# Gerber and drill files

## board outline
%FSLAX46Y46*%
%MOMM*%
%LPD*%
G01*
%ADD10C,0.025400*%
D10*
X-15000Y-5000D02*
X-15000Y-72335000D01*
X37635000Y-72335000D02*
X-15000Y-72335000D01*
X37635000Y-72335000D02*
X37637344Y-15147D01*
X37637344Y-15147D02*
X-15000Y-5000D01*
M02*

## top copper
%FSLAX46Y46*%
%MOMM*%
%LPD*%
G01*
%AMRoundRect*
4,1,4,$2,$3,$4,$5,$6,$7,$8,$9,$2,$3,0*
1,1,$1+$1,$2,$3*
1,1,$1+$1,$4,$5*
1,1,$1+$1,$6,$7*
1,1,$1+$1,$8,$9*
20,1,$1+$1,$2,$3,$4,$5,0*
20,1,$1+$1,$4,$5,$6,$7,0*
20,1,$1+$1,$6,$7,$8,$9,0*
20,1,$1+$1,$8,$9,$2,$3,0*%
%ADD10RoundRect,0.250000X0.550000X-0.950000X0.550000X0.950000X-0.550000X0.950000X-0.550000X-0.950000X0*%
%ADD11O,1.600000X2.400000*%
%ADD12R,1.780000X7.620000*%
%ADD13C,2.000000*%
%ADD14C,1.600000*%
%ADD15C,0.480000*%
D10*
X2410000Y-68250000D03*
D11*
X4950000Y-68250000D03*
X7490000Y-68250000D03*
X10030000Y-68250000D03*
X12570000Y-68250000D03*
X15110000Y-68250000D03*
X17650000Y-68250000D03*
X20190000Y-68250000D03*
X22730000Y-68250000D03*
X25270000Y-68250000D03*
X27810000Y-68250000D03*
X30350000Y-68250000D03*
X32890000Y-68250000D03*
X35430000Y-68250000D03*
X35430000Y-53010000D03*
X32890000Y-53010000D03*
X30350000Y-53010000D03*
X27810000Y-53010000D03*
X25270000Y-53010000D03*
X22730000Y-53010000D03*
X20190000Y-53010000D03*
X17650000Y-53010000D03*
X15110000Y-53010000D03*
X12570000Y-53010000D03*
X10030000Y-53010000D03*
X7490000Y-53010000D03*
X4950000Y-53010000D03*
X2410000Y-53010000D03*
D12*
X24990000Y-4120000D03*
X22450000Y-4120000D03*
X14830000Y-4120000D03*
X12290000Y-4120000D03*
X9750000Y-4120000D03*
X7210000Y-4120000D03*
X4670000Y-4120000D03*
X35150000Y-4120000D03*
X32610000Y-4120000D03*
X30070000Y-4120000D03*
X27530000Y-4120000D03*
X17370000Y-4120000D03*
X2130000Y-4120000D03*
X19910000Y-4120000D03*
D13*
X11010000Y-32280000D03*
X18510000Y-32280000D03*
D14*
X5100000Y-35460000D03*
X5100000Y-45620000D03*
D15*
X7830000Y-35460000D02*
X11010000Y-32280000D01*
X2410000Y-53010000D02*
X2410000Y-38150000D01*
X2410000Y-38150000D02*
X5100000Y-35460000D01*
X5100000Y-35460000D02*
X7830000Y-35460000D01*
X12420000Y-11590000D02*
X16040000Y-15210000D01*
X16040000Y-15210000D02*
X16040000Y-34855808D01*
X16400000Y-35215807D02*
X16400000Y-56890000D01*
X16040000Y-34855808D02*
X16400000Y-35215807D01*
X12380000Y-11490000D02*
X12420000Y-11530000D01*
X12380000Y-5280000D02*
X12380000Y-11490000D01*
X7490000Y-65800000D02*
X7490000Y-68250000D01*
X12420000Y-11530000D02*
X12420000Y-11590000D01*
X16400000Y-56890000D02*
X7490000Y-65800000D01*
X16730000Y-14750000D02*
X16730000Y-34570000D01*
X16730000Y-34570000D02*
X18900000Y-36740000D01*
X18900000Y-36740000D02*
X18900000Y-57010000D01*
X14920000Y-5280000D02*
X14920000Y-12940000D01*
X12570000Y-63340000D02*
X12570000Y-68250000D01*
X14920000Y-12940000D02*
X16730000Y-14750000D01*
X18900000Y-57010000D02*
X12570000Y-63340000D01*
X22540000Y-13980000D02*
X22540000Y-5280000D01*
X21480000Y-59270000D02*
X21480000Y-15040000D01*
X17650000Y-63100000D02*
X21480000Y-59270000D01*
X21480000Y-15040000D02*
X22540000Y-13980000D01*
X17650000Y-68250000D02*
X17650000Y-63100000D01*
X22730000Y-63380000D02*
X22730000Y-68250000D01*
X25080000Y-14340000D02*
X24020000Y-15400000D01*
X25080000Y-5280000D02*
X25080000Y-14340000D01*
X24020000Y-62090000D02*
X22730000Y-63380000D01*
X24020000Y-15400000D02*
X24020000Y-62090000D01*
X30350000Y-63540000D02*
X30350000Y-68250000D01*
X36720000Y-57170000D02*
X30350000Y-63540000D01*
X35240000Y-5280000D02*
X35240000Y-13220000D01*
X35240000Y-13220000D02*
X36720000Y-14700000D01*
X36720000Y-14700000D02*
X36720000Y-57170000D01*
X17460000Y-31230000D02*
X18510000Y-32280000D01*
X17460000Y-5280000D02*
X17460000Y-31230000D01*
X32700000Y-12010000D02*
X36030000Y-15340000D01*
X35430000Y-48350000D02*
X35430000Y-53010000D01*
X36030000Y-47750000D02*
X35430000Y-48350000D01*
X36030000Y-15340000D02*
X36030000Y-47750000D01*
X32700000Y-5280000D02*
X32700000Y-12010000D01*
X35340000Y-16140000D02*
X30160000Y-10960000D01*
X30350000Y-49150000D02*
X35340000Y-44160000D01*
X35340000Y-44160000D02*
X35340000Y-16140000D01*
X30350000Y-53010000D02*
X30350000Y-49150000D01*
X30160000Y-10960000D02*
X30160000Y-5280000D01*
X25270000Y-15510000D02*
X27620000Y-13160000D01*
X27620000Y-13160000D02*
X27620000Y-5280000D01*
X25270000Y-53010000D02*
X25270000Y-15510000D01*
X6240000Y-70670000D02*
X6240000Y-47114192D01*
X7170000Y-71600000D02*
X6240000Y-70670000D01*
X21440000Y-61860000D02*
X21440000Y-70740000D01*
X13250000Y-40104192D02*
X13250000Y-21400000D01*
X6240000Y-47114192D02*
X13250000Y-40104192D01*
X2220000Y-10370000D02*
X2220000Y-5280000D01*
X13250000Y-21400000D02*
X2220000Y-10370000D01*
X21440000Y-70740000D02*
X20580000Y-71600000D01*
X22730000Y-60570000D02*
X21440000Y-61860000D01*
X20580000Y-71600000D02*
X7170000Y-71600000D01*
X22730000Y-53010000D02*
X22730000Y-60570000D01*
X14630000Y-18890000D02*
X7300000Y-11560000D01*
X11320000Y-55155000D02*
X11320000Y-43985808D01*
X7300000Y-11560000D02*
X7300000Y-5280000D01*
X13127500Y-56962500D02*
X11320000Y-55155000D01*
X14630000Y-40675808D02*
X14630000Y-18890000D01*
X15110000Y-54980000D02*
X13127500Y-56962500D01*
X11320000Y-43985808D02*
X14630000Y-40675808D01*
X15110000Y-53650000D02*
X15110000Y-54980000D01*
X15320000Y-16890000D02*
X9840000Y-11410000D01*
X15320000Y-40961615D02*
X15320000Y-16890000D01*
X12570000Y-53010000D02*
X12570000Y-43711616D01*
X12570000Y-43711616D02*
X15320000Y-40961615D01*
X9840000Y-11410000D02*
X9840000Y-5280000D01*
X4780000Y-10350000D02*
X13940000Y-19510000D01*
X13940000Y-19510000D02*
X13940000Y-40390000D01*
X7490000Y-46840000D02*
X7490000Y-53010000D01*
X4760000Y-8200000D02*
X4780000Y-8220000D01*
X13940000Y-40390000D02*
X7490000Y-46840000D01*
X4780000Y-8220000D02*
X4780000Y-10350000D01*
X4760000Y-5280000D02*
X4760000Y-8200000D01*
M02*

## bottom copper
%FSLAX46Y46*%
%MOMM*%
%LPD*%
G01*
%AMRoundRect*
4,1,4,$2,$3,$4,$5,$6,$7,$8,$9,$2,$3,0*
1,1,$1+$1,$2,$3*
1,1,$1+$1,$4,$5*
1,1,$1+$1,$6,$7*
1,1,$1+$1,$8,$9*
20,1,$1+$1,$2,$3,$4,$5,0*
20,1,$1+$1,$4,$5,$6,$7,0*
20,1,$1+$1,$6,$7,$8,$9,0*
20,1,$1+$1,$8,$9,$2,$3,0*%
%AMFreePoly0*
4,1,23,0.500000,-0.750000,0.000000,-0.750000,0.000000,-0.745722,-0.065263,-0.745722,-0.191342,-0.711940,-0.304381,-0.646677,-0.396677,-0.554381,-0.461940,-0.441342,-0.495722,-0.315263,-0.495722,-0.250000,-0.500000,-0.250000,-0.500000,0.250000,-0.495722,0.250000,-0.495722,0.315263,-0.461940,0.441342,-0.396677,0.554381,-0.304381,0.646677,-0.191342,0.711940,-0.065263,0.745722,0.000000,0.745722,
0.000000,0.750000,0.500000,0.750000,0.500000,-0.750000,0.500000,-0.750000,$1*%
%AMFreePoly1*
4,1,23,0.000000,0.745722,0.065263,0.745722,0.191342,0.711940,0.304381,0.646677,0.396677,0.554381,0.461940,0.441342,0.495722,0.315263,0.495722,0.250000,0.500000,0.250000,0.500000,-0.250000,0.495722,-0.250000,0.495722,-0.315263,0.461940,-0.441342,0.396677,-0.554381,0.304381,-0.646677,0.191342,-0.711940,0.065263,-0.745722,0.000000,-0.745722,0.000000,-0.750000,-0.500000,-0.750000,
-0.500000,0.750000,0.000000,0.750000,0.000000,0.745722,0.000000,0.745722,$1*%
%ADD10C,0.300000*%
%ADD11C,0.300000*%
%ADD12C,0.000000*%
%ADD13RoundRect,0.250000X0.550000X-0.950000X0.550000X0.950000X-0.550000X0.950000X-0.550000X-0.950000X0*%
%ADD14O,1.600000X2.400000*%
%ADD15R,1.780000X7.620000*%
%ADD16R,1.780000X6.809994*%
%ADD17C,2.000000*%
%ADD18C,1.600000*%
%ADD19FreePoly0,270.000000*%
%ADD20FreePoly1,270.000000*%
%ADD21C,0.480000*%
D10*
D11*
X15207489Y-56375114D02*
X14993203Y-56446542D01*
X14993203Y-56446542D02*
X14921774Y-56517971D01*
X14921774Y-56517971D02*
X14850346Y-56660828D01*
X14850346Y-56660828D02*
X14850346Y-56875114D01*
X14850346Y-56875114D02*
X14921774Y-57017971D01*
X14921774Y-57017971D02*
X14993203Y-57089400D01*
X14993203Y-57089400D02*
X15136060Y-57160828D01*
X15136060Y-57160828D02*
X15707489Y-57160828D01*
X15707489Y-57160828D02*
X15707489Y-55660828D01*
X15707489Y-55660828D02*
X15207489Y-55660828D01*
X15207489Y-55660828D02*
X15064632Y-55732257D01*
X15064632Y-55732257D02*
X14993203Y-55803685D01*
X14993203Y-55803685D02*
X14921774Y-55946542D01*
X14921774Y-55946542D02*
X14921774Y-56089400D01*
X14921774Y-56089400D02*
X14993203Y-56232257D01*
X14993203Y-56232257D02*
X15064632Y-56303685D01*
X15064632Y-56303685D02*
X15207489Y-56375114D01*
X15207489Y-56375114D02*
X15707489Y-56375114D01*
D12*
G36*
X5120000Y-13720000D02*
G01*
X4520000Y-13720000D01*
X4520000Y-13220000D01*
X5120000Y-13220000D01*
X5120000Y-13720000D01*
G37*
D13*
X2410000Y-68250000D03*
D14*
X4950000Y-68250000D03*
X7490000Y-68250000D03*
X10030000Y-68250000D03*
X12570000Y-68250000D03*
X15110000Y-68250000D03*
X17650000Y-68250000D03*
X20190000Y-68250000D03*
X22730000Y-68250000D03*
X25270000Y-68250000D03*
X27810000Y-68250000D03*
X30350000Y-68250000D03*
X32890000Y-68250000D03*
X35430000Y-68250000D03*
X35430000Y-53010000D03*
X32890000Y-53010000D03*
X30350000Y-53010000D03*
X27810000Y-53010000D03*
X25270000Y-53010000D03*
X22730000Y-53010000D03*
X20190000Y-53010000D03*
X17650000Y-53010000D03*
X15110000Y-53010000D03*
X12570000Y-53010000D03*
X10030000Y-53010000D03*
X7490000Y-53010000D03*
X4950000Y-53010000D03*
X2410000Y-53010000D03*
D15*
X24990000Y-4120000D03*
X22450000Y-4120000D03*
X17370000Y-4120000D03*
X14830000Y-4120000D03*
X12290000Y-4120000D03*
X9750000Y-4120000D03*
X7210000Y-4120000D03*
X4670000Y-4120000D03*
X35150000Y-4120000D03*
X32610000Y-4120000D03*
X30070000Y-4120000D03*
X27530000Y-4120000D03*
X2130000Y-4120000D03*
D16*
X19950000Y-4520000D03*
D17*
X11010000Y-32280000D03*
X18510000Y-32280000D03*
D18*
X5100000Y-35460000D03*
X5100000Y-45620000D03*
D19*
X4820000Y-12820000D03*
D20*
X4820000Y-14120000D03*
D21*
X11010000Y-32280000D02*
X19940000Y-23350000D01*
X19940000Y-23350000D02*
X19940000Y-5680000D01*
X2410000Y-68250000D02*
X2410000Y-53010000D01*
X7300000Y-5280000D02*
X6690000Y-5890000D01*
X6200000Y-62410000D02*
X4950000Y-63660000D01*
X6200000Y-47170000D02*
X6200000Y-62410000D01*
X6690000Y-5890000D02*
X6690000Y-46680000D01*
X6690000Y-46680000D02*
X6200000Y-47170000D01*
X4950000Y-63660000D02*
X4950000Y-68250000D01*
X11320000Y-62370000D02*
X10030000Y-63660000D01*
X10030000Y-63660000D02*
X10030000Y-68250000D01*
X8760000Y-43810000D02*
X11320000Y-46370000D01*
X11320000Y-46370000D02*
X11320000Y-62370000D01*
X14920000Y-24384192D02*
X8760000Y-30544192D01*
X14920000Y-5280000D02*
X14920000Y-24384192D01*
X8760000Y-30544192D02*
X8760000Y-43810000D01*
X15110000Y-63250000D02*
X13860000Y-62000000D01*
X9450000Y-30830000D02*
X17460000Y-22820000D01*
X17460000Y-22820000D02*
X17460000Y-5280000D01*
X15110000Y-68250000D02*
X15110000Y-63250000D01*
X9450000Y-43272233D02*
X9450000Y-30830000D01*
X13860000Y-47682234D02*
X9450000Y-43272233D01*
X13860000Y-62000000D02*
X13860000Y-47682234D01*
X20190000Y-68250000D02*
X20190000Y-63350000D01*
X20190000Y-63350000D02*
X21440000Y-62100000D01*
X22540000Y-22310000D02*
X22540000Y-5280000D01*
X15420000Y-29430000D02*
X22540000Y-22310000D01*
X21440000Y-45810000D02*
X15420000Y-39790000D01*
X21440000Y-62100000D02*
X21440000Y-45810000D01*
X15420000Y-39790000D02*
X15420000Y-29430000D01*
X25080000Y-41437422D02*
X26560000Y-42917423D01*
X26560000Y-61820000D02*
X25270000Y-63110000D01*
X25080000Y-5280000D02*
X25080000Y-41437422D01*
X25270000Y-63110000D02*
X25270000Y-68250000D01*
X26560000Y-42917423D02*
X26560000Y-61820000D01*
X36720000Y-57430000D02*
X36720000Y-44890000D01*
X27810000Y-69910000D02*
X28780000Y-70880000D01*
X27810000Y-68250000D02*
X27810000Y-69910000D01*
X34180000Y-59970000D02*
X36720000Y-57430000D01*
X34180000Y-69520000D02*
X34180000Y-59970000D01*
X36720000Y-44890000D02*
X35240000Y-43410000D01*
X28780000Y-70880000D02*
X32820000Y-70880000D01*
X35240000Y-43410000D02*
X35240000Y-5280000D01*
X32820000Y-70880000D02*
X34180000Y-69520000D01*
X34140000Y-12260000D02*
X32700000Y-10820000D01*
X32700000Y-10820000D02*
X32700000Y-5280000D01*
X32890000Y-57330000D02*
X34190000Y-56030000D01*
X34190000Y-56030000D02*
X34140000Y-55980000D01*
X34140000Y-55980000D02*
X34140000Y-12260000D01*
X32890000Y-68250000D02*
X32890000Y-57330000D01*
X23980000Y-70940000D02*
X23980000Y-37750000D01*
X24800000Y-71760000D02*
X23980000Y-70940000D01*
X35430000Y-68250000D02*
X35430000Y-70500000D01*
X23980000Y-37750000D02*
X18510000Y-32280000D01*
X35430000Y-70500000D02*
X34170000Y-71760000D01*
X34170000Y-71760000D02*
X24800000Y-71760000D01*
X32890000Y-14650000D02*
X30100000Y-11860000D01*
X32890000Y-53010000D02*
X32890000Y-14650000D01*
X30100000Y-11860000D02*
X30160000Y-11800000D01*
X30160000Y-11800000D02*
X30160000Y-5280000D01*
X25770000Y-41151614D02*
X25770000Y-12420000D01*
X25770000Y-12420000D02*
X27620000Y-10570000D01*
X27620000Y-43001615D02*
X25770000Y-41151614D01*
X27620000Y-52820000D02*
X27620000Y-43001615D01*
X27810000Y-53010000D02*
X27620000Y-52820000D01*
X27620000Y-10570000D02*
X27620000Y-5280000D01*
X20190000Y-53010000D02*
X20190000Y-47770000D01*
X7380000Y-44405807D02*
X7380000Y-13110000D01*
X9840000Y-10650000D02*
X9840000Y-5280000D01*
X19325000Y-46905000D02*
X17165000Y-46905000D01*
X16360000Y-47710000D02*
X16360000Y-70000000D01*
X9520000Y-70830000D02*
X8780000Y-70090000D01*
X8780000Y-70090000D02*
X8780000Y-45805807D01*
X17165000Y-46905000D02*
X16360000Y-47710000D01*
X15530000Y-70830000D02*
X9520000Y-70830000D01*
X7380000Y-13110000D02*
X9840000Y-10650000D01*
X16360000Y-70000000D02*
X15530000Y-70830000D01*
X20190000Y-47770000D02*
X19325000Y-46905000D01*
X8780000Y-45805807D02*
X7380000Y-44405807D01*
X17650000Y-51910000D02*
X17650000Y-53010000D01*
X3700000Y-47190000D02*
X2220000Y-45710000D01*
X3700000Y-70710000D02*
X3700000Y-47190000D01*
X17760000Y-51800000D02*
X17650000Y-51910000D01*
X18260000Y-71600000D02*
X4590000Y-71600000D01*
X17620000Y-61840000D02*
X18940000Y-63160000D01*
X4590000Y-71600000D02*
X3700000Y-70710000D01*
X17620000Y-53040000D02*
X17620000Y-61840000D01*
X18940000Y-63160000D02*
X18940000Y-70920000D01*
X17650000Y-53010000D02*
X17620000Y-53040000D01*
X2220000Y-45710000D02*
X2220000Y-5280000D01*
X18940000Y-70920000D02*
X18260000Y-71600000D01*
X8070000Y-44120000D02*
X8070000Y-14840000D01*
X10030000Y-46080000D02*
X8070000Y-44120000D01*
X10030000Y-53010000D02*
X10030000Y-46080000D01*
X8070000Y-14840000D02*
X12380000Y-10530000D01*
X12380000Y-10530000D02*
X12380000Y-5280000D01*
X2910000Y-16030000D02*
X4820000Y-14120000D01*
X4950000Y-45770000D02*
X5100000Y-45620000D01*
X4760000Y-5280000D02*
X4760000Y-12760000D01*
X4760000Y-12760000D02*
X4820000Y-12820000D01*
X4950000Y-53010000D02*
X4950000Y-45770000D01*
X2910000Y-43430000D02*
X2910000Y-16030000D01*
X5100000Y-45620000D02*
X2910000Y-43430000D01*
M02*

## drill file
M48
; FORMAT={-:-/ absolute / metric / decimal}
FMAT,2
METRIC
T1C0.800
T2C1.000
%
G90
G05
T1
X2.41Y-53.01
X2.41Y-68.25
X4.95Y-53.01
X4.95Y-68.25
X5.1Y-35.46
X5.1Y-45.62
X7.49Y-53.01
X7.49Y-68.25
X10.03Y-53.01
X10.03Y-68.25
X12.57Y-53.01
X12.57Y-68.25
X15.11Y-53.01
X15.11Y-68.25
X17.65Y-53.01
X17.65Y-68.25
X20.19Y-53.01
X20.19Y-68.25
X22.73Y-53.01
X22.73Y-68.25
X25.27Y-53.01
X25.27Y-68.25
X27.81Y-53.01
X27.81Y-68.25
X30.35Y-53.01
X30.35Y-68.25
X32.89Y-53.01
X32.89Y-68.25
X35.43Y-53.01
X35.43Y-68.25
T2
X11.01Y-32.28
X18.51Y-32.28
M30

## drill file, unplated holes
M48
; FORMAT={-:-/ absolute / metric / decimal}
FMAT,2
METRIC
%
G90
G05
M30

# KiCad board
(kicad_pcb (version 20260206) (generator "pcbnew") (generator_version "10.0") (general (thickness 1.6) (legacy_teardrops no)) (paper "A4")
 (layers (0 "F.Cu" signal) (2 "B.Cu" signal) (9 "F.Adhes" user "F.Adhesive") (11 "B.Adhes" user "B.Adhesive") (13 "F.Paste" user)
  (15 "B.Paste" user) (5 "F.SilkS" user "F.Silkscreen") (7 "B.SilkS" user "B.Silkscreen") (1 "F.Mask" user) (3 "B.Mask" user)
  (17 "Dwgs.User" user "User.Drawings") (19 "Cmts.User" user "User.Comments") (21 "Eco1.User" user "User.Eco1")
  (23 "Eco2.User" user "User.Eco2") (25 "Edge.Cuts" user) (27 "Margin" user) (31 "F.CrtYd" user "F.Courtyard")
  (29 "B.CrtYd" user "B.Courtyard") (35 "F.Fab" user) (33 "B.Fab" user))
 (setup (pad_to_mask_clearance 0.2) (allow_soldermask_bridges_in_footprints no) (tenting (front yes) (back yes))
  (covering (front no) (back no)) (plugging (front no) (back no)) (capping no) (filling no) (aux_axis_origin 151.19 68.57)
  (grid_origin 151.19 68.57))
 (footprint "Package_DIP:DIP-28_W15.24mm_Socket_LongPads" (layer "F.Cu") (at 153.6 136.82 90)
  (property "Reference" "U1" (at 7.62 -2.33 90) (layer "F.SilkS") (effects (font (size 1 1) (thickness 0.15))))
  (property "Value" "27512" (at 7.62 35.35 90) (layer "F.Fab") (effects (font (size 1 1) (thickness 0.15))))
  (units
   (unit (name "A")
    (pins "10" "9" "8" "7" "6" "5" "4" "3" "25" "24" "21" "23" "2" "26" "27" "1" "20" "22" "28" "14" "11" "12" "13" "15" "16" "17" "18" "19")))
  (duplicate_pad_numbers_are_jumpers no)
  (pad "1" thru_hole roundrect (at 0 0 90) (size 2.4 1.6) (drill 0.8) (layers "*.Cu" "*.Mask") (remove_unused_layers no)
   (roundrect_rratio 0.15625) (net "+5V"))
  (pad "2" thru_hole oval (at 0 2.54 90) (size 2.4 1.6) (drill 0.8) (layers "*.Cu" "*.Mask") (remove_unused_layers no) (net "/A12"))
  (pad "3" thru_hole oval (at 0 5.08 90) (size 2.4 1.6) (drill 0.8) (layers "*.Cu" "*.Mask") (remove_unused_layers no) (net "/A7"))
  (pad "4" thru_hole oval (at 0 7.62 90) (size 2.4 1.6) (drill 0.8) (layers "*.Cu" "*.Mask") (remove_unused_layers no) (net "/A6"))
  (pad "5" thru_hole oval (at 0 10.16 90) (size 2.4 1.6) (drill 0.8) (layers "*.Cu" "*.Mask") (remove_unused_layers no) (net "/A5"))
  (pad "6" thru_hole oval (at 0 12.7 90) (size 2.4 1.6) (drill 0.8) (layers "*.Cu" "*.Mask") (remove_unused_layers no) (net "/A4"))
  (pad "7" thru_hole oval (at 0 15.24 90) (size 2.4 1.6) (drill 0.8) (layers "*.Cu" "*.Mask") (remove_unused_layers no) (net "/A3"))
  (pad "8" thru_hole oval (at 0 17.78 90) (size 2.4 1.6) (drill 0.8) (layers "*.Cu" "*.Mask") (remove_unused_layers no) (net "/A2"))
  (pad "9" thru_hole oval (at 0 20.32 90) (size 2.4 1.6) (drill 0.8) (layers "*.Cu" "*.Mask") (remove_unused_layers no) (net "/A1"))
  (pad "10" thru_hole oval (at 0 22.86 90) (size 2.4 1.6) (drill 0.8) (layers "*.Cu" "*.Mask") (remove_unused_layers no) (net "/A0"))
  (pad "11" thru_hole oval (at 0 25.4 90) (size 2.4 1.6) (drill 0.8) (layers "*.Cu" "*.Mask") (remove_unused_layers no) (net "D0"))
  (pad "12" thru_hole oval (at 0 27.94 90) (size 2.4 1.6) (drill 0.8) (layers "*.Cu" "*.Mask") (remove_unused_layers no) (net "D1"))
  (pad "13" thru_hole oval (at 0 30.48 90) (size 2.4 1.6) (drill 0.8) (layers "*.Cu" "*.Mask") (remove_unused_layers no) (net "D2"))
  (pad "14" thru_hole oval (at 0 33.02 90) (size 2.4 1.6) (drill 0.8) (layers "*.Cu" "*.Mask") (remove_unused_layers no) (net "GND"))
  (pad "15" thru_hole oval (at 15.24 33.02 90) (size 2.4 1.6) (drill 0.8) (layers "*.Cu" "*.Mask") (remove_unused_layers no) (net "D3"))
  (pad "16" thru_hole oval (at 15.24 30.48 90) (size 2.4 1.6) (drill 0.8) (layers "*.Cu" "*.Mask") (remove_unused_layers no) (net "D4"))
  (pad "17" thru_hole oval (at 15.24 27.94 90) (size 2.4 1.6) (drill 0.8) (layers "*.Cu" "*.Mask") (remove_unused_layers no) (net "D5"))
  (pad "18" thru_hole oval (at 15.24 25.4 90) (size 2.4 1.6) (drill 0.8) (layers "*.Cu" "*.Mask") (remove_unused_layers no) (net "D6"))
  (pad "19" thru_hole oval (at 15.24 22.86 90) (size 2.4 1.6) (drill 0.8) (layers "*.Cu" "*.Mask") (remove_unused_layers no) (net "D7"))
  (pad "20" thru_hole oval (at 15.24 20.32 90) (size 2.4 1.6) (drill 0.8) (layers "*.Cu" "*.Mask") (remove_unused_layers no)
   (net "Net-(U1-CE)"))
  (pad "21" thru_hole oval (at 15.24 17.78 90) (size 2.4 1.6) (drill 0.8) (layers "*.Cu" "*.Mask") (remove_unused_layers no) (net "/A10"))
  (pad "22" thru_hole oval (at 15.24 15.24 90) (size 2.4 1.6) (drill 0.8) (layers "*.Cu" "*.Mask") (remove_unused_layers no)
   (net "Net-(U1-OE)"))
  (pad "23" thru_hole oval (at 15.24 12.7 90) (size 2.4 1.6) (drill 0.8) (layers "*.Cu" "*.Mask") (remove_unused_layers no) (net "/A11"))
  (pad "24" thru_hole oval (at 15.24 10.16 90) (size 2.4 1.6) (drill 0.8) (layers "*.Cu" "*.Mask") (remove_unused_layers no) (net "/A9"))
  (pad "25" thru_hole oval (at 15.24 7.62 90) (size 2.4 1.6) (drill 0.8) (layers "*.Cu" "*.Mask") (remove_unused_layers no) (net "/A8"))
  (pad "26" thru_hole oval (at 15.24 5.08 90) (size 2.4 1.6) (drill 0.8) (layers "*.Cu" "*.Mask") (remove_unused_layers no) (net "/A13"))
  (pad "27" thru_hole oval (at 15.24 2.54 90) (size 2.4 1.6) (drill 0.8) (layers "*.Cu" "*.Mask") (remove_unused_layers no) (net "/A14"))
  (pad "28" thru_hole oval (at 15.24 0 90) (size 2.4 1.6) (drill 0.8) (layers "*.Cu" "*.Mask") (remove_unused_layers no) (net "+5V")))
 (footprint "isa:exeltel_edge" (layer "F.Cu") (at 186.34 72.69)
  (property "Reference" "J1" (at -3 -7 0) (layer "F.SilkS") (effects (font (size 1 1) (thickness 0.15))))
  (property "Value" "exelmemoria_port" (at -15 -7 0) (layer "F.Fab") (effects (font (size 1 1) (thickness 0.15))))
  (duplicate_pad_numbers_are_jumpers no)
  (pad "AD0" connect rect (at -10.16 0) (size 1.78 7.62) (layers "B.Cu" "B.Mask") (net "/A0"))
  (pad "AD1" connect rect (at -10.16 0) (size 1.78 7.62) (layers "F.Cu" "F.Mask") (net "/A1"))
  (pad "AD2" connect rect (at -12.7 0) (size 1.78 7.62) (layers "B.Cu" "B.Mask") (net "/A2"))
  (pad "AD3" connect rect (at -12.7 0) (size 1.78 7.62) (layers "F.Cu" "F.Mask") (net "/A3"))
  (pad "AD4" connect rect (at -17.78 0) (size 1.78 7.62) (layers "B.Cu" "B.Mask") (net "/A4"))
  (pad "AD5" connect rect (at -20.32 0) (size 1.78 7.62) (layers "F.Cu" "F.Mask") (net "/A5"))
  (pad "AD6" connect rect (at -20.32 0) (size 1.78 7.62) (layers "B.Cu" "B.Mask") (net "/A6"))
  (pad "AD7" connect rect (at -22.86 0) (size 1.78 7.62) (layers "F.Cu" "F.Mask") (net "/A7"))
  (pad "AD8" connect rect (at -22.86 0) (size 1.78 7.62) (layers "B.Cu" "B.Mask") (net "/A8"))
  (pad "AD9" connect rect (at -25.4 0) (size 1.78 7.62) (layers "F.Cu" "F.Mask") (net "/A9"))
  (pad "AD10" connect rect (at -25.4 0) (size 1.78 7.62) (layers "B.Cu" "B.Mask") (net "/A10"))
  (pad "AD11" connect rect (at -27.94 0) (size 1.78 7.62) (layers "F.Cu" "F.Mask") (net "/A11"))
  (pad "AD12" connect rect (at -27.94 0) (size 1.78 7.62) (layers "B.Cu" "B.Mask") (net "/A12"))
  (pad "AD13" connect rect (at -30.48 0) (size 1.78 7.62) (layers "F.Cu" "F.Mask") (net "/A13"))
  (pad "AD14" connect rect (at -30.48 0) (size 1.78 7.62) (layers "B.Cu" "B.Mask") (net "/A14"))
  (pad "DB0" connect rect (at 0 0) (size 1.78 7.62) (layers "B.Cu" "B.Mask") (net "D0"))
  (pad "DB1" connect rect (at 0 0) (size 1.78 7.62) (layers "F.Cu" "F.Mask") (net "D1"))
  (pad "DB2" connect rect (at -2.54 0) (size 1.78 7.62) (layers "B.Cu" "B.Mask") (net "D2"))
  (pad "DB3" connect rect (at -2.54 0) (size 1.78 7.62) (layers "F.Cu" "F.Mask") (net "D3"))
  (pad "DB4" connect rect (at -5.08 0) (size 1.78 7.62) (layers "B.Cu" "B.Mask") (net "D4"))
  (pad "DB5" connect rect (at -5.08 0) (size 1.78 7.62) (layers "F.Cu" "F.Mask") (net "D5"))
  (pad "DB6" connect rect (at -7.62 0) (size 1.78 7.62) (layers "B.Cu" "B.Mask") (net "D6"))
  (pad "DB7" connect rect (at -7.62 0) (size 1.78 7.62) (layers "F.Cu" "F.Mask") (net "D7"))
  (pad "GND" connect rect (at -17.78 0) (size 1.78 7.62) (layers "F.Cu" "F.Mask") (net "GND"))
  (pad "NROMCS" connect rect (at -33.02 0) (size 1.78 7.62) (layers "F.Cu" "F.Mask") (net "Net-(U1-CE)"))
  (pad "NROMOE" connect rect (at -33.02 0) (size 1.78 7.62) (layers "B.Cu" "B.Mask") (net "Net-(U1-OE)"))
  (pad "SPARIN7" connect rect (at -15.24 0) (size 1.78 7.62) (layers "F.Cu" "F.Mask") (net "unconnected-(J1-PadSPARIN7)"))
  (pad "VCC" connect rect (at -15.2 0.4) (size 1.78 6.809994) (layers "B.Cu" "B.Mask") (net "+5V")))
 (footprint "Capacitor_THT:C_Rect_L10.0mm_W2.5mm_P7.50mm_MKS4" (layer "F.Cu") (at 162.2 100.85)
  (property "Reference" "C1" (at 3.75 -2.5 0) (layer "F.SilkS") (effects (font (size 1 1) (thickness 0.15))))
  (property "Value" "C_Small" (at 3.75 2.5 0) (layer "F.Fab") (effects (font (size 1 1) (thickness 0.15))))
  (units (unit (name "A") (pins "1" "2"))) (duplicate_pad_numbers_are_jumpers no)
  (pad "1" thru_hole circle (at 0 0) (size 2 2) (drill 1) (layers "*.Cu" "*.Mask") (remove_unused_layers no) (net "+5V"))
  (pad "2" thru_hole circle (at 7.5 0) (size 2 2) (drill 1) (layers "*.Cu" "*.Mask") (remove_unused_layers no) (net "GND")))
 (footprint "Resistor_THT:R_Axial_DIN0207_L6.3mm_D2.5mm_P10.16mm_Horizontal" (layer "F.Cu") (at 156.29 104.03 -90)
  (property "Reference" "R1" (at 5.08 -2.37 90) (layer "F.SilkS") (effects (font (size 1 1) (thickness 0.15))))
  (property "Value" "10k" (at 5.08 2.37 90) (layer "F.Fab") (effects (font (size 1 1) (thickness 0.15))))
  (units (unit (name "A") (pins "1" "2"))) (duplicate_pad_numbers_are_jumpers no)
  (pad "1" thru_hole circle (at 0 0 270) (size 1.6 1.6) (drill 0.8) (layers "*.Cu" "*.Mask") (remove_unused_layers no) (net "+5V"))
  (pad "2" thru_hole circle (at 10.16 0 270) (size 1.6 1.6) (drill 0.8) (layers "*.Cu" "*.Mask") (remove_unused_layers no) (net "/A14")))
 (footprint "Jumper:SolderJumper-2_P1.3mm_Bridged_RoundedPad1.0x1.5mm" (layer "B.Cu") (at 156.01 82.04 -90)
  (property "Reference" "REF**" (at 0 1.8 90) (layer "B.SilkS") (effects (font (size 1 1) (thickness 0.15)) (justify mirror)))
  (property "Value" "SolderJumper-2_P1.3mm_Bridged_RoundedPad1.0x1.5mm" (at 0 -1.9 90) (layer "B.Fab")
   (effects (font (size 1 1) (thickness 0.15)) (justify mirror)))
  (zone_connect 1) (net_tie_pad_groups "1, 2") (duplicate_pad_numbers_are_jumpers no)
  (fp_poly (pts (xy 0.25 0.3) (xy -0.25 0.3) (xy -0.25 -0.3) (xy 0.25 -0.3)) (stroke (width 0) (type solid)) (fill yes) (layer "B.Cu"))
  (pad "1" smd custom (at -0.65 0 270) (size 1 0.5) (layers "B.Cu" "B.Mask") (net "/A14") (zone_connect 2) (thermal_bridge_angle 45)
   (options (clearance outline) (anchor rect)) (primitives))
  (pad "2" smd custom (at 0.65 0 270) (size 1 0.5) (layers "B.Cu" "B.Mask") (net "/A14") (zone_connect 2) (thermal_bridge_angle 45)
   (options (clearance outline) (anchor rect)) (primitives)))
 (gr_line (start 151.175 68.575) (end 151.175 140.905) (stroke (width 0.0254) (type default)) (layer "Edge.Cuts"))
 (gr_line (start 188.825 140.905) (end 151.175 140.905) (stroke (width 0.0254) (type default)) (layer "Edge.Cuts"))
 (gr_line (start 188.825 140.905) (end 188.827344 68.585147) (stroke (width 0.0254) (type default)) (layer "Edge.Cuts"))
 (gr_line (start 188.827344 68.585147) (end 151.175 68.575) (stroke (width 0.0254) (type default)) (layer "Edge.Cuts"))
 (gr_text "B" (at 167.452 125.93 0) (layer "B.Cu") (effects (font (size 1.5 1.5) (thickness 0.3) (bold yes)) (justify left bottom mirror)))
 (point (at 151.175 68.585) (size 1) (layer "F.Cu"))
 (segment (start 159.02 104.03) (end 162.2 100.85) (width 0.48) (layer "F.Cu") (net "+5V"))
 (segment (start 153.6 121.58) (end 153.6 106.72) (width 0.48) (layer "F.Cu") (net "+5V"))
 (segment (start 153.6 106.72) (end 156.29 104.03) (width 0.48) (layer "F.Cu") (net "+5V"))
 (segment (start 156.29 104.03) (end 159.02 104.03) (width 0.48) (layer "F.Cu") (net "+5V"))
 (segment (start 162.2 100.85) (end 171.13 91.92) (width 0.48) (layer "B.Cu") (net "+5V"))
 (segment (start 171.13 91.92) (end 171.13 74.25) (width 0.48) (layer "B.Cu") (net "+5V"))
 (segment (start 153.6 136.82) (end 153.6 121.58) (width 0.48) (layer "B.Cu") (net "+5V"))
 (segment (start 158.49 73.85) (end 157.88 74.46) (width 0.48) (layer "B.Cu") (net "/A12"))
 (segment (start 157.39 130.98) (end 156.14 132.23) (width 0.48) (layer "B.Cu") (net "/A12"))
 (segment (start 157.39 115.74) (end 157.39 130.98) (width 0.48) (layer "B.Cu") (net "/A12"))
 (segment (start 157.88 74.46) (end 157.88 115.25) (width 0.48) (layer "B.Cu") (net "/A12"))
 (segment (start 157.88 115.25) (end 157.39 115.74) (width 0.48) (layer "B.Cu") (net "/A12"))
 (segment (start 156.14 132.23) (end 156.14 136.82) (width 0.48) (layer "B.Cu") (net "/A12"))
 (segment (start 163.61 80.16) (end 167.23 83.78) (width 0.48) (layer "F.Cu") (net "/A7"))
 (segment (start 167.23 83.78) (end 167.23 103.425808) (width 0.48) (layer "F.Cu") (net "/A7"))
 (segment (start 167.59 103.785807) (end 167.59 125.46) (width 0.48) (layer "F.Cu") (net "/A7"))
 (segment (start 167.23 103.425808) (end 167.59 103.785807) (width 0.48) (layer "F.Cu") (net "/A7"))
 (segment (start 163.57 80.06) (end 163.61 80.1) (width 0.48) (layer "F.Cu") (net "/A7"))
 (segment (start 163.57 73.85) (end 163.57 80.06) (width 0.48) (layer "F.Cu") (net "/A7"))
 (segment (start 158.68 134.37) (end 158.68 136.82) (width 0.48) (layer "F.Cu") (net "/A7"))
 (segment (start 163.61 80.1) (end 163.61 80.16) (width 0.48) (layer "F.Cu") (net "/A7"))
 (segment (start 167.59 125.46) (end 158.68 134.37) (width 0.48) (layer "F.Cu") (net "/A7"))
 (segment (start 162.51 130.94) (end 161.22 132.23) (width 0.48) (layer "B.Cu") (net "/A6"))
 (segment (start 161.22 132.23) (end 161.22 136.82) (width 0.48) (layer "B.Cu") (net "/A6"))
 (segment (start 159.95 112.38) (end 162.51 114.94) (width 0.48) (layer "B.Cu") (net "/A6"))
 (segment (start 162.51 114.94) (end 162.51 130.94) (width 0.48) (layer "B.Cu") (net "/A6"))
 (segment (start 166.11 92.954192) (end 159.95 99.114192) (width 0.48) (layer "B.Cu") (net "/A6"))
 (segment (start 166.11 73.85) (end 166.11 92.954192) (width 0.48) (layer "B.Cu") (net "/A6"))
 (segment (start 159.95 99.114192) (end 159.95 112.38) (width 0.48) (layer "B.Cu") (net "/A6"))
 (segment (start 167.92 83.32) (end 167.92 103.14) (width 0.48) (layer "F.Cu") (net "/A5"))
 (segment (start 167.92 103.14) (end 170.09 105.31) (width 0.48) (layer "F.Cu") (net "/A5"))
 (segment (start 170.09 105.31) (end 170.09 125.58) (width 0.48) (layer "F.Cu") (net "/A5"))
 (segment (start 166.11 73.85) (end 166.11 81.51) (width 0.48) (layer "F.Cu") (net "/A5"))
 (segment (start 163.76 131.91) (end 163.76 136.82) (width 0.48) (layer "F.Cu") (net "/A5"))
 (segment (start 166.11 81.51) (end 167.92 83.32) (width 0.48) (layer "F.Cu") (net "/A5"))
 (segment (start 170.09 125.58) (end 163.76 131.91) (width 0.48) (layer "F.Cu") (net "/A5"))
 (segment (start 166.3 131.82) (end 165.05 130.57) (width 0.48) (layer "B.Cu") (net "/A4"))
 (segment (start 160.64 99.4) (end 168.65 91.39) (width 0.48) (layer "B.Cu") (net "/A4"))
 (segment (start 168.65 91.39) (end 168.65 73.85) (width 0.48) (layer "B.Cu") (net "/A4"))
 (segment (start 166.3 136.82) (end 166.3 131.82) (width 0.48) (layer "B.Cu") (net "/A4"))
 (segment (start 160.64 111.842233) (end 160.64 99.4) (width 0.48) (layer "B.Cu") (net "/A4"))
 (segment (start 165.05 116.252234) (end 160.64 111.842233) (width 0.48) (layer "B.Cu") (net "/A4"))
 (segment (start 165.05 130.57) (end 165.05 116.252234) (width 0.48) (layer "B.Cu") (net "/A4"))
 (segment (start 173.73 82.55) (end 173.73 73.85) (width 0.48) (layer "F.Cu") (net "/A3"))
 (segment (start 172.67 127.84) (end 172.67 83.61) (width 0.48) (layer "F.Cu") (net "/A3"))
 (segment (start 168.84 131.67) (end 172.67 127.84) (width 0.48) (layer "F.Cu") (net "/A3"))
 (segment (start 172.67 83.61) (end 173.73 82.55) (width 0.48) (layer "F.Cu") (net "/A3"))
 (segment (start 168.84 136.82) (end 168.84 131.67) (width 0.48) (layer "F.Cu") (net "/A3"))
 (segment (start 171.38 136.82) (end 171.38 131.92) (width 0.48) (layer "B.Cu") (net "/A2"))
 (segment (start 171.38 131.92) (end 172.63 130.67) (width 0.48) (layer "B.Cu") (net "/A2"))
 (segment (start 173.73 90.88) (end 173.73 73.85) (width 0.48) (layer "B.Cu") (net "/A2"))
 (segment (start 166.61 98) (end 173.73 90.88) (width 0.48) (layer "B.Cu") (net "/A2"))
 (segment (start 172.63 114.38) (end 166.61 108.36) (width 0.48) (layer "B.Cu") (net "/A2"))
 (segment (start 172.63 130.67) (end 172.63 114.38) (width 0.48) (layer "B.Cu") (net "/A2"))
 (segment (start 166.61 108.36) (end 166.61 98) (width 0.48) (layer "B.Cu") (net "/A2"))
 (segment (start 173.92 131.95) (end 173.92 136.82) (width 0.48) (layer "F.Cu") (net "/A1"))
 (segment (start 176.27 82.91) (end 175.21 83.97) (width 0.48) (layer "F.Cu") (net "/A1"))
 (segment (start 176.27 73.85) (end 176.27 82.91) (width 0.48) (layer "F.Cu") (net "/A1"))
 (segment (start 175.21 130.66) (end 173.92 131.95) (width 0.48) (layer "F.Cu") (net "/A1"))
 (segment (start 175.21 83.97) (end 175.21 130.66) (width 0.48) (layer "F.Cu") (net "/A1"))
 (segment (start 176.27 110.007422) (end 177.75 111.487423) (width 0.48) (layer "B.Cu") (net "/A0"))
 (segment (start 177.75 130.39) (end 176.46 131.68) (width 0.48) (layer "B.Cu") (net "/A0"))
 (segment (start 176.27 73.85) (end 176.27 110.007422) (width 0.48) (layer "B.Cu") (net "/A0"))
 (segment (start 176.46 131.68) (end 176.46 136.82) (width 0.48) (layer "B.Cu") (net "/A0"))
 (segment (start 177.75 111.487423) (end 177.75 130.39) (width 0.48) (layer "B.Cu") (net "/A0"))
 (segment (start 187.91 126) (end 187.91 113.46) (width 0.48) (layer "B.Cu") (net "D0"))
 (segment (start 179 138.48) (end 179.97 139.45) (width 0.48) (layer "B.Cu") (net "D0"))
 (segment (start 179 136.82) (end 179 138.48) (width 0.48) (layer "B.Cu") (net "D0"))
 (segment (start 185.37 128.54) (end 187.91 126) (width 0.48) (layer "B.Cu") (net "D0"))
 (segment (start 185.37 138.09) (end 185.37 128.54) (width 0.48) (layer "B.Cu") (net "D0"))
 (segment (start 187.91 113.46) (end 186.43 111.98) (width 0.48) (layer "B.Cu") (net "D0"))
 (segment (start 179.97 139.45) (end 184.01 139.45) (width 0.48) (layer "B.Cu") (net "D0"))
 (segment (start 186.43 111.98) (end 186.43 73.85) (width 0.48) (layer "B.Cu") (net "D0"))
 (segment (start 184.01 139.45) (end 185.37 138.09) (width 0.48) (layer "B.Cu") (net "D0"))
 (segment (start 181.54 132.11) (end 181.54 136.82) (width 0.48) (layer "F.Cu") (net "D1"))
 (segment (start 187.91 125.74) (end 181.54 132.11) (width 0.48) (layer "F.Cu") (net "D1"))
 (segment (start 186.43 73.85) (end 186.43 81.79) (width 0.48) (layer "F.Cu") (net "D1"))
 (segment (start 186.43 81.79) (end 187.91 83.27) (width 0.48) (layer "F.Cu") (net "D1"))
 (segment (start 187.91 83.27) (end 187.91 125.74) (width 0.48) (layer "F.Cu") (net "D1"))
 (segment (start 185.33 80.83) (end 183.89 79.39) (width 0.48) (layer "B.Cu") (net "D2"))
 (segment (start 183.89 79.39) (end 183.89 73.85) (width 0.48) (layer "B.Cu") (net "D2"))
 (segment (start 184.08 125.9) (end 185.38 124.6) (width 0.48) (layer "B.Cu") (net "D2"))
 (segment (start 185.38 124.6) (end 185.33 124.55) (width 0.48) (layer "B.Cu") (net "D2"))
 (segment (start 185.33 124.55) (end 185.33 80.83) (width 0.48) (layer "B.Cu") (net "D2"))
 (segment (start 184.08 136.82) (end 184.08 125.9) (width 0.48) (layer "B.Cu") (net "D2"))
 (segment (start 168.65 99.8) (end 169.7 100.85) (width 0.48) (layer "F.Cu") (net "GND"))
 (segment (start 168.65 73.85) (end 168.65 99.8) (width 0.48) (layer "F.Cu") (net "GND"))
 (segment (start 175.17 139.51) (end 175.17 106.32) (width 0.48) (layer "B.Cu") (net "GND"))
 (segment (start 175.99 140.33) (end 175.17 139.51) (width 0.48) (layer "B.Cu") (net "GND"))
 (segment (start 186.62 136.82) (end 186.62 139.07) (width 0.48) (layer "B.Cu") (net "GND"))
 (segment (start 175.17 106.32) (end 169.7 100.85) (width 0.48) (layer "B.Cu") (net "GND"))
 (segment (start 186.62 139.07) (end 185.36 140.33) (width 0.48) (layer "B.Cu") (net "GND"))
 (segment (start 185.36 140.33) (end 175.99 140.33) (width 0.48) (layer "B.Cu") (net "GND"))
 (segment (start 183.89 80.58) (end 187.22 83.91) (width 0.48) (layer "F.Cu") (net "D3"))
 (segment (start 186.62 116.92) (end 186.62 121.58) (width 0.48) (layer "F.Cu") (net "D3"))
 (segment (start 187.22 116.32) (end 186.62 116.92) (width 0.48) (layer "F.Cu") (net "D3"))
 (segment (start 187.22 83.91) (end 187.22 116.32) (width 0.48) (layer "F.Cu") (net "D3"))
 (segment (start 183.89 73.85) (end 183.89 80.58) (width 0.48) (layer "F.Cu") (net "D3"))
 (segment (start 184.08 83.22) (end 181.29 80.43) (width 0.48) (layer "B.Cu") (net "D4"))
 (segment (start 184.08 121.58) (end 184.08 83.22) (width 0.48) (layer "B.Cu") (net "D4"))
 (segment (start 181.29 80.43) (end 181.35 80.37) (width 0.48) (layer "B.Cu") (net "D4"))
 (segment (start 181.35 80.37) (end 181.35 73.85) (width 0.48) (layer "B.Cu") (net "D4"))
 (segment (start 186.53 84.71) (end 181.35 79.53) (width 0.48) (layer "F.Cu") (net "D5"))
 (segment (start 181.54 117.72) (end 186.53 112.73) (width 0.48) (layer "F.Cu") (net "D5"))
 (segment (start 186.53 112.73) (end 186.53 84.71) (width 0.48) (layer "F.Cu") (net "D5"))
 (segment (start 181.54 121.58) (end 181.54 117.72) (width 0.48) (layer "F.Cu") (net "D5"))
 (segment (start 181.35 79.53) (end 181.35 73.85) (width 0.48) (layer "F.Cu") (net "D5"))
 (segment (start 176.96 109.721614) (end 176.96 80.99) (width 0.48) (layer "B.Cu") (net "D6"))
 (segment (start 176.96 80.99) (end 178.81 79.14) (width 0.48) (layer "B.Cu") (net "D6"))
 (segment (start 178.81 111.571615) (end 176.96 109.721614) (width 0.48) (layer "B.Cu") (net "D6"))
 (segment (start 178.81 121.39) (end 178.81 111.571615) (width 0.48) (layer "B.Cu") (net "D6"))
 (segment (start 179 121.58) (end 178.81 121.39) (width 0.48) (layer "B.Cu") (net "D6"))
 (segment (start 178.81 79.14) (end 178.81 73.85) (width 0.48) (layer "B.Cu") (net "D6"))
 (segment (start 176.46 84.08) (end 178.81 81.73) (width 0.48) (layer "F.Cu") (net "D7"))
 (segment (start 178.81 81.73) (end 178.81 73.85) (width 0.48) (layer "F.Cu") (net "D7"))
 (segment (start 176.46 121.58) (end 176.46 84.08) (width 0.48) (layer "F.Cu") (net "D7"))
 (segment (start 157.43 139.24) (end 157.43 115.684192) (width 0.48) (layer "F.Cu") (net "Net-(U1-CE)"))
 (segment (start 158.36 140.17) (end 157.43 139.24) (width 0.48) (layer "F.Cu") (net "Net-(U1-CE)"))
 (segment (start 172.63 130.43) (end 172.63 139.31) (width 0.48) (layer "F.Cu") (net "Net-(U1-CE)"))
 (segment (start 164.44 108.674192) (end 164.44 89.97) (width 0.48) (layer "F.Cu") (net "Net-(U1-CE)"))
 (segment (start 157.43 115.684192) (end 164.44 108.674192) (width 0.48) (layer "F.Cu") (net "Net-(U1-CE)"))
 (segment (start 153.41 78.94) (end 153.41 73.85) (width 0.48) (layer "F.Cu") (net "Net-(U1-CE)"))
 (segment (start 164.44 89.97) (end 153.41 78.94) (width 0.48) (layer "F.Cu") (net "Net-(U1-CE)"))
 (segment (start 172.63 139.31) (end 171.77 140.17) (width 0.48) (layer "F.Cu") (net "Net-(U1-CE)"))
 (segment (start 173.92 129.14) (end 172.63 130.43) (width 0.48) (layer "F.Cu") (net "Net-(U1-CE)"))
 (segment (start 171.77 140.17) (end 158.36 140.17) (width 0.48) (layer "F.Cu") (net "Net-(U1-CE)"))
 (segment (start 173.92 121.58) (end 173.92 129.14) (width 0.48) (layer "F.Cu") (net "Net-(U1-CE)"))
 (segment (start 171.38 121.58) (end 171.38 116.34) (width 0.48) (layer "B.Cu") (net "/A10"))
 (segment (start 158.57 112.975807) (end 158.57 81.68) (width 0.48) (layer "B.Cu") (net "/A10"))
 (segment (start 161.03 79.22) (end 161.03 73.85) (width 0.48) (layer "B.Cu") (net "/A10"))
 (segment (start 170.515 115.475) (end 168.355 115.475) (width 0.48) (layer "B.Cu") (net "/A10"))
 (segment (start 167.55 116.28) (end 167.55 138.57) (width 0.48) (layer "B.Cu") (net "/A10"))
 (segment (start 160.71 139.4) (end 159.97 138.66) (width 0.48) (layer "B.Cu") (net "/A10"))
 (segment (start 159.97 138.66) (end 159.97 114.375807) (width 0.48) (layer "B.Cu") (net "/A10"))
 (segment (start 168.355 115.475) (end 167.55 116.28) (width 0.48) (layer "B.Cu") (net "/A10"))
 (segment (start 166.72 139.4) (end 160.71 139.4) (width 0.48) (layer "B.Cu") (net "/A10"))
 (segment (start 158.57 81.68) (end 161.03 79.22) (width 0.48) (layer "B.Cu") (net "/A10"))
 (segment (start 167.55 138.57) (end 166.72 139.4) (width 0.48) (layer "B.Cu") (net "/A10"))
 (segment (start 171.38 116.34) (end 170.515 115.475) (width 0.48) (layer "B.Cu") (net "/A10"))
 (segment (start 159.97 114.375807) (end 158.57 112.975807) (width 0.48) (layer "B.Cu") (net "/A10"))
 (segment (start 168.84 120.48) (end 168.84 121.58) (width 0.48) (layer "B.Cu") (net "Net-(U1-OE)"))
 (segment (start 154.89 115.76) (end 153.41 114.28) (width 0.48) (layer "B.Cu") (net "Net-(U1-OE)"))
 (segment (start 154.89 139.28) (end 154.89 115.76) (width 0.48) (layer "B.Cu") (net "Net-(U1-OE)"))
 (segment (start 168.95 120.37) (end 168.84 120.48) (width 0.48) (layer "B.Cu") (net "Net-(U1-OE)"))
 (segment (start 169.45 140.17) (end 155.78 140.17) (width 0.48) (layer "B.Cu") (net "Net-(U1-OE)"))
 (segment (start 168.81 130.41) (end 170.13 131.73) (width 0.48) (layer "B.Cu") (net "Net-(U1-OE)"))
 (segment (start 155.78 140.17) (end 154.89 139.28) (width 0.48) (layer "B.Cu") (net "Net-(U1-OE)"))
 (segment (start 168.81 121.61) (end 168.81 130.41) (width 0.48) (layer "B.Cu") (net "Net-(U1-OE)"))
 (segment (start 170.13 131.73) (end 170.13 139.49) (width 0.48) (layer "B.Cu") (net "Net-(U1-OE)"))
 (segment (start 168.84 121.58) (end 168.81 121.61) (width 0.48) (layer "B.Cu") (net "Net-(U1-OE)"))
 (segment (start 153.41 114.28) (end 153.41 73.85) (width 0.48) (layer "B.Cu") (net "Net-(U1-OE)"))
 (segment (start 170.13 139.49) (end 169.45 140.17) (width 0.48) (layer "B.Cu") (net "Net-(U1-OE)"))
 (segment (start 165.82 87.46) (end 158.49 80.13) (width 0.48) (layer "F.Cu") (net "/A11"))
 (segment (start 162.51 123.725) (end 162.51 112.555808) (width 0.48) (layer "F.Cu") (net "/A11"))
 (segment (start 158.49 80.13) (end 158.49 73.85) (width 0.48) (layer "F.Cu") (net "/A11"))
 (segment (start 164.3175 125.5325) (end 162.51 123.725) (width 0.48) (layer "F.Cu") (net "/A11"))
 (segment (start 165.82 109.245808) (end 165.82 87.46) (width 0.48) (layer "F.Cu") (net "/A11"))
 (segment (start 166.3 123.55) (end 164.3175 125.5325) (width 0.48) (layer "F.Cu") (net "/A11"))
 (segment (start 162.51 112.555808) (end 165.82 109.245808) (width 0.48) (layer "F.Cu") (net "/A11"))
 (segment (start 166.3 122.22) (end 166.3 123.55) (width 0.48) (layer "F.Cu") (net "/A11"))
 (segment (start 166.51 85.46) (end 161.03 79.98) (width 0.48) (layer "F.Cu") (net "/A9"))
 (segment (start 166.51 109.531615) (end 166.51 85.46) (width 0.48) (layer "F.Cu") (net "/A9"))
 (segment (start 163.76 121.58) (end 163.76 112.281616) (width 0.48) (layer "F.Cu") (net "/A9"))
 (segment (start 163.76 112.281616) (end 166.51 109.531615) (width 0.48) (layer "F.Cu") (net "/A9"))
 (segment (start 161.03 79.98) (end 161.03 73.85) (width 0.48) (layer "F.Cu") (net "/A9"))
 (segment (start 159.26 112.69) (end 159.26 83.41) (width 0.48) (layer "B.Cu") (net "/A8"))
 (segment (start 161.22 114.65) (end 159.26 112.69) (width 0.48) (layer "B.Cu") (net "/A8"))
 (segment (start 161.22 121.58) (end 161.22 114.65) (width 0.48) (layer "B.Cu") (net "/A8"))
 (segment (start 159.26 83.41) (end 163.57 79.1) (width 0.48) (layer "B.Cu") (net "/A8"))
 (segment (start 163.57 79.1) (end 163.57 73.85) (width 0.48) (layer "B.Cu") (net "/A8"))
 (segment (start 155.97 78.92) (end 165.13 88.08) (width 0.48) (layer "F.Cu") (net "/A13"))
 (segment (start 165.13 88.08) (end 165.13 108.96) (width 0.48) (layer "F.Cu") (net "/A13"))
 (segment (start 158.68 115.41) (end 158.68 121.58) (width 0.48) (layer "F.Cu") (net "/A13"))
 (segment (start 155.95 76.77) (end 155.97 76.79) (width 0.48) (layer "F.Cu") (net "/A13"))
 (segment (start 165.13 108.96) (end 158.68 115.41) (width 0.48) (layer "F.Cu") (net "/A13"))
 (segment (start 155.97 76.79) (end 155.97 78.92) (width 0.48) (layer "F.Cu") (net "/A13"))
 (segment (start 155.95 73.85) (end 155.95 76.77) (width 0.48) (layer "F.Cu") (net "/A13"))
 (segment (start 154.1 84.6) (end 156.01 82.69) (width 0.48) (layer "B.Cu") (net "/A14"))
 (segment (start 156.14 114.34) (end 156.29 114.19) (width 0.48) (layer "B.Cu") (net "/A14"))
 (segment (start 155.95 73.85) (end 155.95 81.33) (width 0.48) (layer "B.Cu") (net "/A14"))
 (segment (start 155.95 81.33) (end 156.01 81.39) (width 0.48) (layer "B.Cu") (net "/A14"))
 (segment (start 156.14 121.58) (end 156.14 114.34) (width 0.48) (layer "B.Cu") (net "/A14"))
 (segment (start 154.1 112) (end 154.1 84.6) (width 0.48) (layer "B.Cu") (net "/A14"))
 (segment (start 156.29 114.19) (end 154.1 112) (width 0.48) (layer "B.Cu") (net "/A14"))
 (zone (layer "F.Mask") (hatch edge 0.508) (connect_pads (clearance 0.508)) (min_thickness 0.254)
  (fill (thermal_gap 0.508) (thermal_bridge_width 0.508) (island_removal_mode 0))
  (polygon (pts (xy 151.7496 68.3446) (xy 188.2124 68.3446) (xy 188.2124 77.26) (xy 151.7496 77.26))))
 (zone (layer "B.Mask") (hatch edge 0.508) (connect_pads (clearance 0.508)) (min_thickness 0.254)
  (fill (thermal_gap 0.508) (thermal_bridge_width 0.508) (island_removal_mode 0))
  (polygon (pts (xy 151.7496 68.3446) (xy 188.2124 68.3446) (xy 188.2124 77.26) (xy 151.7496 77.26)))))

